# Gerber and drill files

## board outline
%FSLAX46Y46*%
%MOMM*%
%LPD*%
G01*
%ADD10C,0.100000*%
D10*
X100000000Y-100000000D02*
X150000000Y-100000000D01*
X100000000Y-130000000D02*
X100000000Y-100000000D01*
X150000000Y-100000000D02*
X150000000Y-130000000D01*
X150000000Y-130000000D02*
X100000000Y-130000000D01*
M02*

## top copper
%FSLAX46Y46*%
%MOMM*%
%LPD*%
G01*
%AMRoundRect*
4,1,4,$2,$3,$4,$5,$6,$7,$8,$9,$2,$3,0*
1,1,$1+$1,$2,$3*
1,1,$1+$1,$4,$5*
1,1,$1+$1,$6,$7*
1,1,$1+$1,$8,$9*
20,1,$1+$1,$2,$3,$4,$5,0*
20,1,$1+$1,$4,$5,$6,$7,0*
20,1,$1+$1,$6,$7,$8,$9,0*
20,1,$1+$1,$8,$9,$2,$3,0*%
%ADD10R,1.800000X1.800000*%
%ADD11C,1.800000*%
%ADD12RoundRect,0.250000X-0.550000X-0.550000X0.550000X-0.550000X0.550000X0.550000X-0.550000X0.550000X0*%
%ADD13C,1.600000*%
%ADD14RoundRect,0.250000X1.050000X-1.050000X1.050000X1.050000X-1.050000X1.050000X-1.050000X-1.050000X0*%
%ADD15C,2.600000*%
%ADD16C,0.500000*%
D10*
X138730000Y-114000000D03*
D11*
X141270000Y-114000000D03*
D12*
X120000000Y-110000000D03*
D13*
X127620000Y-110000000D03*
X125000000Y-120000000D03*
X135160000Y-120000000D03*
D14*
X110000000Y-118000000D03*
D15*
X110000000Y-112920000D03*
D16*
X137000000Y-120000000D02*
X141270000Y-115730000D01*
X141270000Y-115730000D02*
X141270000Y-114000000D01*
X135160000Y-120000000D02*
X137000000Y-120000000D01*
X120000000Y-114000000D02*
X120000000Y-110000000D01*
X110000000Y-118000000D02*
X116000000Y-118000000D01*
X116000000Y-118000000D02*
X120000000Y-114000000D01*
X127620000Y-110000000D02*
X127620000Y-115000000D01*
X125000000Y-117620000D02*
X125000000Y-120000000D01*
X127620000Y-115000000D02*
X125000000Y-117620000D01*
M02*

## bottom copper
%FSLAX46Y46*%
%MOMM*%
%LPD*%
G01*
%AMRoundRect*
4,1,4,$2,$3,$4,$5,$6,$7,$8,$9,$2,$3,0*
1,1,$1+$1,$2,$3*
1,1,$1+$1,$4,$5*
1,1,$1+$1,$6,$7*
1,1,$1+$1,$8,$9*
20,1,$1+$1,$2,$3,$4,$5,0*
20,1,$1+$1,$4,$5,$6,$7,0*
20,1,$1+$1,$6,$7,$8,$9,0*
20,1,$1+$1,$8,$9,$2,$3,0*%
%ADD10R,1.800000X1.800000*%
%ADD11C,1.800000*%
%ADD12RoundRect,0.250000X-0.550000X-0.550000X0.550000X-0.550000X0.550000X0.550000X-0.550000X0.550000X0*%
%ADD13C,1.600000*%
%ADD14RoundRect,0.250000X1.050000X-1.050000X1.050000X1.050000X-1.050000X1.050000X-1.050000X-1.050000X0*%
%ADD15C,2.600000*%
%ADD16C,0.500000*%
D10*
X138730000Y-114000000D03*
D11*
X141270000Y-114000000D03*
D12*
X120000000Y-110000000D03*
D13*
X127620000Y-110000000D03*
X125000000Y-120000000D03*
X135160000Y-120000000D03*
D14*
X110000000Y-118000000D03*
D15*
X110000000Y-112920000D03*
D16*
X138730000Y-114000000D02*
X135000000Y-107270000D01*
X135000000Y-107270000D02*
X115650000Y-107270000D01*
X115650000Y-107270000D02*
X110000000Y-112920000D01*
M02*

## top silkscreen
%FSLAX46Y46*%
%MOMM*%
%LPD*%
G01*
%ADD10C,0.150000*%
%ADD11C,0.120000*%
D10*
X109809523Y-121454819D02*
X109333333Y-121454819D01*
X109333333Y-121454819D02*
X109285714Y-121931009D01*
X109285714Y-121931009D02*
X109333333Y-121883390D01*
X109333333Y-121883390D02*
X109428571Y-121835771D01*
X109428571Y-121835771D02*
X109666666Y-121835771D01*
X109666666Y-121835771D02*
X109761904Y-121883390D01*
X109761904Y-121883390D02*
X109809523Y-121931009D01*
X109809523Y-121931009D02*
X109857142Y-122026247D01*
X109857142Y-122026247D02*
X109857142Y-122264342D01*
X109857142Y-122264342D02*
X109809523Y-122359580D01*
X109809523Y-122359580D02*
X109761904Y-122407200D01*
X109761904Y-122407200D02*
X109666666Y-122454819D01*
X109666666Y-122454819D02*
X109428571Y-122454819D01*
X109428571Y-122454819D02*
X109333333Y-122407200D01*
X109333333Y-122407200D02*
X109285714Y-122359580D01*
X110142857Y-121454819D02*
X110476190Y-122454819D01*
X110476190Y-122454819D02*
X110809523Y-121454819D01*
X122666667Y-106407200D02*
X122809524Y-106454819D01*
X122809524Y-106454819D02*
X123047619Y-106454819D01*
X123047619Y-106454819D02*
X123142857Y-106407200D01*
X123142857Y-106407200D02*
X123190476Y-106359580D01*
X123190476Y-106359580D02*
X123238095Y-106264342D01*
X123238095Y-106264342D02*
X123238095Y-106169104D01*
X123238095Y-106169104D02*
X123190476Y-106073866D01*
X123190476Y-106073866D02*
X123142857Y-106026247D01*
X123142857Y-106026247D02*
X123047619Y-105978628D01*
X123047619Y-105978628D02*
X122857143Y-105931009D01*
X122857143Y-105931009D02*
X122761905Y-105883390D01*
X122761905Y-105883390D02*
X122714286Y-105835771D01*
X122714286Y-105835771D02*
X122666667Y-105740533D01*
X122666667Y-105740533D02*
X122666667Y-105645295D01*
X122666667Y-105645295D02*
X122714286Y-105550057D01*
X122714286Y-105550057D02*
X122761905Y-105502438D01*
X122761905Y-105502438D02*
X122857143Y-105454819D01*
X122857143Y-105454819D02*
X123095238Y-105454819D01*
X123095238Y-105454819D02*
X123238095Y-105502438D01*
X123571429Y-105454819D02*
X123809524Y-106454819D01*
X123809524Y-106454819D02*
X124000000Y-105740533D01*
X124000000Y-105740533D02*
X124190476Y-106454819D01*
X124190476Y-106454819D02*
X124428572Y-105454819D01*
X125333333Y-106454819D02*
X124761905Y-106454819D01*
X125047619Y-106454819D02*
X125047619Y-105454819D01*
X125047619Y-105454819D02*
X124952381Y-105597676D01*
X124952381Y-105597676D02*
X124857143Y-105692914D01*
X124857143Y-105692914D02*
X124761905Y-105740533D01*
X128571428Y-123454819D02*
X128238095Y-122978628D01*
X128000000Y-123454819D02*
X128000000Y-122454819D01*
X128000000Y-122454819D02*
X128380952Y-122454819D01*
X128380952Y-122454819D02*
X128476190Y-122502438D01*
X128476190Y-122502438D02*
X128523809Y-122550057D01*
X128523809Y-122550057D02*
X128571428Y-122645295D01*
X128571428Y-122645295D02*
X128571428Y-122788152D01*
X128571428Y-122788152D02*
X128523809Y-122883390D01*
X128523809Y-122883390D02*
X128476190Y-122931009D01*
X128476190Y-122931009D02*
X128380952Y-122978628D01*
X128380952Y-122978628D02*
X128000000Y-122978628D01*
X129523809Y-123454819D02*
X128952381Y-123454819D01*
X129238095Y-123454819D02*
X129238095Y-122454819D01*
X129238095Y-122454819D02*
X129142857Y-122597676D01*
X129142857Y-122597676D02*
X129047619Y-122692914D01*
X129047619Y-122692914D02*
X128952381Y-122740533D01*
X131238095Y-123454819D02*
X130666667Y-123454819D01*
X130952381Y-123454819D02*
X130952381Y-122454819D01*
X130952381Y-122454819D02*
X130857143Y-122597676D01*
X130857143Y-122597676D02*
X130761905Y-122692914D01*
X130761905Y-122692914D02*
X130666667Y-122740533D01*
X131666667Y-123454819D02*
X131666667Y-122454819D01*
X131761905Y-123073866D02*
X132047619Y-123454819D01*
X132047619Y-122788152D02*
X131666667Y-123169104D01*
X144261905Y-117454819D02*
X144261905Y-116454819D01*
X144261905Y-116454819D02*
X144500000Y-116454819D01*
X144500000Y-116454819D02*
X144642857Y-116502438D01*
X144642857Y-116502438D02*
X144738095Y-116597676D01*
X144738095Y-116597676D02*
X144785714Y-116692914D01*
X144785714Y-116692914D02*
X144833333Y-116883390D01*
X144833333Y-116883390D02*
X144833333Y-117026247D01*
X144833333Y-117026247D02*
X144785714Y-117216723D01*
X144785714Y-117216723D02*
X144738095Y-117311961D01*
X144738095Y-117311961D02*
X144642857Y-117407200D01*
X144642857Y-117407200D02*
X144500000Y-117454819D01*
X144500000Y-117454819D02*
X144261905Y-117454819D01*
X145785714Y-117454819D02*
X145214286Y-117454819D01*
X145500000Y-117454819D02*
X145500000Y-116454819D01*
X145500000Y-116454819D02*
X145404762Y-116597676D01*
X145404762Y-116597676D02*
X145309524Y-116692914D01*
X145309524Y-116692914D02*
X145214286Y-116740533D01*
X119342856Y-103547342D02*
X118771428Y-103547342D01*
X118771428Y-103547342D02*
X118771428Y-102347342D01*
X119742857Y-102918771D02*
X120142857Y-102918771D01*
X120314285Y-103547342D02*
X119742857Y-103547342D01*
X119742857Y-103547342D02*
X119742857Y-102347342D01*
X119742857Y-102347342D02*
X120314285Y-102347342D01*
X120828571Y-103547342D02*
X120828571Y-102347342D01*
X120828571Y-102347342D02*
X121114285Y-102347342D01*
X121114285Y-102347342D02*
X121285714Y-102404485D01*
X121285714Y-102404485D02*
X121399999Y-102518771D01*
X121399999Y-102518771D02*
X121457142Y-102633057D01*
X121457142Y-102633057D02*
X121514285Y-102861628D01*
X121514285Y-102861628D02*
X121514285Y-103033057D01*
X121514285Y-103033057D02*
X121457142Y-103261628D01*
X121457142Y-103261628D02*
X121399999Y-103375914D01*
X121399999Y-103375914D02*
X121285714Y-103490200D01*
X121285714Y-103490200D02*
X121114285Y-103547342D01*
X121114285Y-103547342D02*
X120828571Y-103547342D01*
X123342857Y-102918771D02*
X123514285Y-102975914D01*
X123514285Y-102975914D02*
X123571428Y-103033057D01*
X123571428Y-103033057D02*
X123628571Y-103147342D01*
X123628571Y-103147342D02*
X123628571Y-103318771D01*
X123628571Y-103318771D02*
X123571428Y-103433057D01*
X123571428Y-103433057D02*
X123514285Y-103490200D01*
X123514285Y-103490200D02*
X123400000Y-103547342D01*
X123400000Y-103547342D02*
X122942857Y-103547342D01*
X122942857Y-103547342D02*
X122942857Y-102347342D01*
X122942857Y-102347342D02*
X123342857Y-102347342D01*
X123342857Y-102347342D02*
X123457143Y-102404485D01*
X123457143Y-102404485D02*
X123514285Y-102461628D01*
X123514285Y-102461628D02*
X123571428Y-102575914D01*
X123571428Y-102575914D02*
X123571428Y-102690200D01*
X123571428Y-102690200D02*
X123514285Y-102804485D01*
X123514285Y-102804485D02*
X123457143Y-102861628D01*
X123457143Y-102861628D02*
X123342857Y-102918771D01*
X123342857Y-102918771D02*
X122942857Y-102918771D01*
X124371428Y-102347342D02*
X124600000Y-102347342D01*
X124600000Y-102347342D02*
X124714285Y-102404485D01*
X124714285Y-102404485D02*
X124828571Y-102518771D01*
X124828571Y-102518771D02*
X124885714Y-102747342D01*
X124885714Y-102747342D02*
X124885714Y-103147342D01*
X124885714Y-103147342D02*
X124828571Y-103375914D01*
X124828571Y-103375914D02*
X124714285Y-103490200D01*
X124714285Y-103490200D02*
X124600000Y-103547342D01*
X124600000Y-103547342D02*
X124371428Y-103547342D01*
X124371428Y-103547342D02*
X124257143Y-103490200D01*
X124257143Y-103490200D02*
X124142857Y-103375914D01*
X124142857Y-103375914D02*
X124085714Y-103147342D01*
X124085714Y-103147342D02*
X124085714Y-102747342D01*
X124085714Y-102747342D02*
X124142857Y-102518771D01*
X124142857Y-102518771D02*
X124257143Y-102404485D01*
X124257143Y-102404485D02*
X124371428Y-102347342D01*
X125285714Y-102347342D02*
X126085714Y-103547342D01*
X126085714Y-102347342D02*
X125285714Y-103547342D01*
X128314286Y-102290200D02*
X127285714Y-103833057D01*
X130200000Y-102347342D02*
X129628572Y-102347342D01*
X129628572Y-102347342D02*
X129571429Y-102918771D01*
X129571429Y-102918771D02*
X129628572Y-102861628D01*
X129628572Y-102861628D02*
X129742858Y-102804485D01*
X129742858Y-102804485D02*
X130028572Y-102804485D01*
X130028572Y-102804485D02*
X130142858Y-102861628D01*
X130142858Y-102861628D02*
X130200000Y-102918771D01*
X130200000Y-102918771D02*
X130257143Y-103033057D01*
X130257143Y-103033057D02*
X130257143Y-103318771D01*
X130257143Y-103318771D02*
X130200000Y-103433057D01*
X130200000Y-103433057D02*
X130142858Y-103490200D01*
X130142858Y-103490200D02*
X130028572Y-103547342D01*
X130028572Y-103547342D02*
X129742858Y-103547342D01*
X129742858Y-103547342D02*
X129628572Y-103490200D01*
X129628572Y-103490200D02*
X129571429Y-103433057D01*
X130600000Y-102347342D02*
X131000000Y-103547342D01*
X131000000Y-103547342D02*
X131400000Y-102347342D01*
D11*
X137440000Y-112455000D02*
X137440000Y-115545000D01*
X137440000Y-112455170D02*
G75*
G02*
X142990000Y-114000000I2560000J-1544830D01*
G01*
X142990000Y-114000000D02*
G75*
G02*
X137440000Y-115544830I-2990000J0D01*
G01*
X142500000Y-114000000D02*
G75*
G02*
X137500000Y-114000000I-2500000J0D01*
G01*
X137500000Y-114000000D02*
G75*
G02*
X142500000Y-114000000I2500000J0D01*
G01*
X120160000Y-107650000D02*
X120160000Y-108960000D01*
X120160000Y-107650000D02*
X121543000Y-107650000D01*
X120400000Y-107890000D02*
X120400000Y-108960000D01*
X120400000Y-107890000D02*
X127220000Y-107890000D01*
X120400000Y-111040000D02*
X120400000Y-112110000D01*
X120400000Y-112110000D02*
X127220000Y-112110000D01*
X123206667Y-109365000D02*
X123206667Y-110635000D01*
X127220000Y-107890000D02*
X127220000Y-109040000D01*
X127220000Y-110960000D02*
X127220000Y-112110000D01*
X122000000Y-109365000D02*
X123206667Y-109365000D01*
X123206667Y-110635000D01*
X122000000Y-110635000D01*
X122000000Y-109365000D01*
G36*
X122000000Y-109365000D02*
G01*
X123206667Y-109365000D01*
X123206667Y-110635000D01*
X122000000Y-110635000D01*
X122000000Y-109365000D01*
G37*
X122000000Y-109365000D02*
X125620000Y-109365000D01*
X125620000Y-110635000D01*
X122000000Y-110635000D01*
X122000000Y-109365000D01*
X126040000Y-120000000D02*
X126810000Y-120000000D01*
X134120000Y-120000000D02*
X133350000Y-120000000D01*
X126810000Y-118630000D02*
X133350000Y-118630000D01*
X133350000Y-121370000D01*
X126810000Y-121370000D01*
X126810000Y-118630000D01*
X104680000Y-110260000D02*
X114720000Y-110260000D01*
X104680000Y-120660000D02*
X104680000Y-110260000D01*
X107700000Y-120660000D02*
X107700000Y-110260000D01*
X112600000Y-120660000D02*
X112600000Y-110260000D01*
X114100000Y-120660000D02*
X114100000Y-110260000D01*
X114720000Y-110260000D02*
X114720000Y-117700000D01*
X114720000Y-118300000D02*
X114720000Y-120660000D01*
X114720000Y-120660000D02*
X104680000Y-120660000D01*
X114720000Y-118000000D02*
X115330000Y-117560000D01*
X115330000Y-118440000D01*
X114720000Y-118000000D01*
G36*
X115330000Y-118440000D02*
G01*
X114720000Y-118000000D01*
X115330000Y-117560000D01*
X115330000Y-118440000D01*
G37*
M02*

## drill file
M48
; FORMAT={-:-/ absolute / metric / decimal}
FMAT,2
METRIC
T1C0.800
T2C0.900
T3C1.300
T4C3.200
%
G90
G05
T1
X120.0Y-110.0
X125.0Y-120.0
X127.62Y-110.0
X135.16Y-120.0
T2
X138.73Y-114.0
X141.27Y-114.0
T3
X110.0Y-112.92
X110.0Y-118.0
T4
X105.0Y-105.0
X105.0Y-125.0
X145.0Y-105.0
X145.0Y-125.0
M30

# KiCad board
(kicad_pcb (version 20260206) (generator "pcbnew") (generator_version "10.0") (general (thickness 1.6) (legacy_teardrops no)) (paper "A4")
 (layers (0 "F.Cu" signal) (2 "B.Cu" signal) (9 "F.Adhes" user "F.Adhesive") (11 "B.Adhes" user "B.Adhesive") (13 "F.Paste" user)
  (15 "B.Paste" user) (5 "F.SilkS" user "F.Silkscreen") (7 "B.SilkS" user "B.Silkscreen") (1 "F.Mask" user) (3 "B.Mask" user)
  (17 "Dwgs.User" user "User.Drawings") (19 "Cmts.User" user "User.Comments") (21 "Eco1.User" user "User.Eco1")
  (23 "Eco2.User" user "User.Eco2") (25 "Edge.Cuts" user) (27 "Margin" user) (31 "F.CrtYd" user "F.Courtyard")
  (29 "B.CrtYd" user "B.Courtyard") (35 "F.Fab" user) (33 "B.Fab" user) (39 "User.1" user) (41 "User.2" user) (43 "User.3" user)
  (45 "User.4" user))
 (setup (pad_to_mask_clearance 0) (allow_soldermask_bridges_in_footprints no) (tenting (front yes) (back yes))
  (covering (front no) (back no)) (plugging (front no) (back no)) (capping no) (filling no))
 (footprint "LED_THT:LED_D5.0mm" (layer "F.Cu") (at 138.73 114)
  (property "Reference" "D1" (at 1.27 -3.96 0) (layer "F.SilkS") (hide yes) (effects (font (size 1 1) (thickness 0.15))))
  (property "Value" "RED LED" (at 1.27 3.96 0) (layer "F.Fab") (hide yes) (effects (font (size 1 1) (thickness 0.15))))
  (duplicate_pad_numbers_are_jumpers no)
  (fp_line (start -1.29 -1.545) (end -1.29 1.545) (stroke (width 0.12) (type solid)) (layer "F.SilkS"))
  (fp_arc (start -1.29 -1.54483) (mid 2.071779 -2.880495) (end 4.26 0) (stroke (width 0.12) (type solid)) (layer "F.SilkS"))
  (fp_arc (start 4.26 0) (mid 2.071779 2.880495) (end -1.29 1.54483) (stroke (width 0.12) (type solid)) (layer "F.SilkS"))
  (fp_circle (center 1.27 0) (end 3.77 0) (stroke (width 0.12) (type solid)) (fill no) (layer "F.SilkS"))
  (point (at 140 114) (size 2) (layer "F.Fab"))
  (pad "1" thru_hole rect (at 0 0) (size 1.8 1.8) (drill 0.9) (layers "*.Cu" "*.Mask") (remove_unused_layers no) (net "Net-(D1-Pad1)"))
  (pad "2" thru_hole circle (at 2.54 0) (size 1.8 1.8) (drill 0.9) (layers "*.Cu" "*.Mask") (remove_unused_layers no) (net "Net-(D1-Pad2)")))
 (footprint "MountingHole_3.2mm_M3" (layer "F.Cu") (at 145 105)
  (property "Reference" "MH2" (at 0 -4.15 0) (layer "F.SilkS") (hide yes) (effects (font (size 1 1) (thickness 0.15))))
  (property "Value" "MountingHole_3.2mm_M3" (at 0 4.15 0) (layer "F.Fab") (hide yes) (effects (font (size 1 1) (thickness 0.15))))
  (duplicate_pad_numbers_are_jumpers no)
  (pad "" np_thru_hole circle (at 0 0) (size 3.2 3.2) (drill 3.2) (layers "*.Cu" "*.Mask")))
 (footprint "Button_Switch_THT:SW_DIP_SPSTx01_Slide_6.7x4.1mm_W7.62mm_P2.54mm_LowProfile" (layer "F.Cu") (at 120 110)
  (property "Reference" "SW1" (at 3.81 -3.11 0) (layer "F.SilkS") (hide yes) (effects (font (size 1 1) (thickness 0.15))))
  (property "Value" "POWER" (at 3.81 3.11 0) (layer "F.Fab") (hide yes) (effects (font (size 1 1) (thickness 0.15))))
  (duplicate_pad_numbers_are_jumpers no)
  (fp_line (start 0.16 -2.35) (end 0.16 -1.04) (stroke (width 0.12) (type solid)) (layer "F.SilkS"))
  (fp_line (start 0.16 -2.35) (end 1.543 -2.35) (stroke (width 0.12) (type solid)) (layer "F.SilkS"))
  (fp_line (start 0.4 -2.11) (end 0.4 -1.04) (stroke (width 0.12) (type solid)) (layer "F.SilkS"))
  (fp_line (start 0.4 -2.11) (end 7.22 -2.11) (stroke (width 0.12) (type solid)) (layer "F.SilkS"))
  (fp_line (start 0.4 1.04) (end 0.4 2.11) (stroke (width 0.12) (type solid)) (layer "F.SilkS"))
  (fp_line (start 0.4 2.11) (end 7.22 2.11) (stroke (width 0.12) (type solid)) (layer "F.SilkS"))
  (fp_line (start 3.206667 -0.635) (end 3.206667 0.635) (stroke (width 0.12) (type solid)) (layer "F.SilkS"))
  (fp_line (start 7.22 -2.11) (end 7.22 -0.96) (stroke (width 0.12) (type solid)) (layer "F.SilkS"))
  (fp_line (start 7.22 0.96) (end 7.22 2.11) (stroke (width 0.12) (type solid)) (layer "F.SilkS"))
  (fp_rect (start 2 -0.635) (end 3.206667 0.635) (stroke (width 0.12) (type solid)) (fill yes) (layer "F.SilkS"))
  (fp_rect (start 2 -0.635) (end 5.62 0.635) (stroke (width 0.12) (type solid)) (fill no) (layer "F.SilkS"))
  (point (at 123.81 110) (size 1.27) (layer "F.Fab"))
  (pad "1" thru_hole roundrect (at 0 0) (size 1.6 1.6) (drill 0.8) (layers "*.Cu" "*.Mask") (remove_unused_layers no)
   (roundrect_rratio 0.15625) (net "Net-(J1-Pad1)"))
  (pad "2" thru_hole circle (at 7.62 0) (size 1.6 1.6) (drill 0.8) (layers "*.Cu" "*.Mask") (remove_unused_layers no) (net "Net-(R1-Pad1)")))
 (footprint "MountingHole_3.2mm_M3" (layer "F.Cu") (at 145 125)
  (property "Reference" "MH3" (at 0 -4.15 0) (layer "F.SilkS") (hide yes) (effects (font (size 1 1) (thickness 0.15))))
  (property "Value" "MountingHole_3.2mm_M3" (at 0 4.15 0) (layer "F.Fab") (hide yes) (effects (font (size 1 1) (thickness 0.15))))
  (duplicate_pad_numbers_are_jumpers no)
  (pad "" np_thru_hole circle (at 0 0) (size 3.2 3.2) (drill 3.2) (layers "*.Cu" "*.Mask")))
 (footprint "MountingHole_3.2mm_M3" (layer "F.Cu") (at 105 125)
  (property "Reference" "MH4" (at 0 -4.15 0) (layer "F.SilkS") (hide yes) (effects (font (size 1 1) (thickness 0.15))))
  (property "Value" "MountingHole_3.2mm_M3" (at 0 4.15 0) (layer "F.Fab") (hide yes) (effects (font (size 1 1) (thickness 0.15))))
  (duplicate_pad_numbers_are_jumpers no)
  (pad "" np_thru_hole circle (at 0 0) (size 3.2 3.2) (drill 3.2) (layers "*.Cu" "*.Mask")))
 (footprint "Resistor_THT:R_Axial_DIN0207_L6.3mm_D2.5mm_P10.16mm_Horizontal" (layer "F.Cu") (at 125 120)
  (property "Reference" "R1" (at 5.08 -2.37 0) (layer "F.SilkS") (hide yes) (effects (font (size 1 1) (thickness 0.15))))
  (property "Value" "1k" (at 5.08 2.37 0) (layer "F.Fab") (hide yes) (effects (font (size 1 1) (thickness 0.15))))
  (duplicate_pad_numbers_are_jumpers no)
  (fp_line (start 1.04 0) (end 1.81 0) (stroke (width 0.12) (type solid)) (layer "F.SilkS"))
  (fp_line (start 9.12 0) (end 8.35 0) (stroke (width 0.12) (type solid)) (layer "F.SilkS"))
  (fp_rect (start 1.81 -1.37) (end 8.35 1.37) (stroke (width 0.12) (type solid)) (fill no) (layer "F.SilkS"))
  (pad "1" thru_hole circle (at 0 0) (size 1.6 1.6) (drill 0.8) (layers "*.Cu" "*.Mask") (remove_unused_layers no) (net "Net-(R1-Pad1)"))
  (pad "2" thru_hole circle (at 10.16 0) (size 1.6 1.6) (drill 0.8) (layers "*.Cu" "*.Mask") (remove_unused_layers no) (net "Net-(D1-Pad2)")))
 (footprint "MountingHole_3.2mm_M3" (layer "F.Cu") (at 105 105)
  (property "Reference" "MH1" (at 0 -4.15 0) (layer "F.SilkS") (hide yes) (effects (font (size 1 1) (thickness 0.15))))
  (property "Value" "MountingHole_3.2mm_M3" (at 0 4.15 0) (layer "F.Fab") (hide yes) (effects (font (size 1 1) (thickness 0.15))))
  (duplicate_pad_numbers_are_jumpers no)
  (pad "" np_thru_hole circle (at 0 0) (size 3.2 3.2) (drill 3.2) (layers "*.Cu" "*.Mask")))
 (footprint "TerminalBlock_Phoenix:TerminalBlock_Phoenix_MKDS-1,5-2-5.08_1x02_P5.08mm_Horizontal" (layer "F.Cu") (at 110 118 90)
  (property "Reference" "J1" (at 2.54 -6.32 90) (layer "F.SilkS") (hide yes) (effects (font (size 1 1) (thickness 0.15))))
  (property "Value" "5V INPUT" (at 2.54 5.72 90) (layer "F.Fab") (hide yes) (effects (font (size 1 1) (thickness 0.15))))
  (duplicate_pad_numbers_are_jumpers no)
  (fp_line (start 7.74 -5.32) (end 7.74 4.72) (stroke (width 0.12) (type solid)) (layer "F.SilkS"))
  (fp_line (start -2.66 -5.32) (end 7.74 -5.32) (stroke (width 0.12) (type solid)) (layer "F.SilkS"))
  (fp_line (start -2.66 -2.3) (end 7.74 -2.3) (stroke (width 0.12) (type solid)) (layer "F.SilkS"))
  (fp_line (start -2.66 2.6) (end 7.74 2.6) (stroke (width 0.12) (type solid)) (layer "F.SilkS"))
  (fp_line (start -2.66 4.1) (end 7.74 4.1) (stroke (width 0.12) (type solid)) (layer "F.SilkS"))
  (fp_line (start 7.74 4.72) (end 0.3 4.72) (stroke (width 0.12) (type solid)) (layer "F.SilkS"))
  (fp_line (start -0.3 4.72) (end -2.66 4.72) (stroke (width 0.12) (type solid)) (layer "F.SilkS"))
  (fp_line (start -2.66 4.72) (end -2.66 -5.32) (stroke (width 0.12) (type solid)) (layer "F.SilkS"))
  (fp_poly (pts (xy 0 4.72) (xy 0.44 5.33) (xy -0.44 5.33)) (stroke (width 0.12) (type solid)) (fill yes) (layer "F.SilkS"))
  (pad "1" thru_hole roundrect (at 0 0 90) (size 2.6 2.6) (drill 1.3) (layers "*.Cu" "*.Mask") (remove_unused_layers no)
   (roundrect_rratio 0.096154) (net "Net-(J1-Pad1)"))
  (pad "2" thru_hole circle (at 5.08 0 90) (size 2.6 2.6) (drill 1.3) (layers "*.Cu" "*.Mask") (remove_unused_layers no)
   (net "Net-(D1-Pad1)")))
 (gr_line (start 100 100) (end 150 100) (stroke (width 0.1) (type default)) (layer "Edge.Cuts"))
 (gr_line (start 100 130) (end 100 100) (stroke (width 0.1) (type default)) (layer "Edge.Cuts"))
 (gr_line (start 150 100) (end 150 130) (stroke (width 0.1) (type default)) (layer "Edge.Cuts"))
 (gr_line (start 150 130) (end 100 130) (stroke (width 0.1) (type default)) (layer "Edge.Cuts"))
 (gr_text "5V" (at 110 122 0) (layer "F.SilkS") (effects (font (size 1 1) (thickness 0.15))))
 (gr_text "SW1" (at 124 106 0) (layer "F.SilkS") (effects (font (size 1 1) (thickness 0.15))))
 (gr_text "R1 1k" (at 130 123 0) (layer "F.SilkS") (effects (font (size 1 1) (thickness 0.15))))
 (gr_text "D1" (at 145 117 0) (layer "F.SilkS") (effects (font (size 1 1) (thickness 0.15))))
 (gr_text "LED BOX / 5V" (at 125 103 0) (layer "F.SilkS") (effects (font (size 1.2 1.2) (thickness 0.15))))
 (segment (start 138.73 114) (end 135 107.27) (width 0.5) (layer "B.Cu") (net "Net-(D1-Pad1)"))
 (segment (start 135 107.27) (end 115.65 107.27) (width 0.5) (layer "B.Cu") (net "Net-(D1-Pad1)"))
 (segment (start 115.65 107.27) (end 110 112.92) (width 0.5) (layer "B.Cu") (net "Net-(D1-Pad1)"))
 (segment (start 137 120) (end 141.27 115.73) (width 0.5) (layer "F.Cu") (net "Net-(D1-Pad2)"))
 (segment (start 141.27 115.73) (end 141.27 114) (width 0.5) (layer "F.Cu") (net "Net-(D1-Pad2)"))
 (segment (start 135.16 120) (end 137 120) (width 0.5) (layer "F.Cu") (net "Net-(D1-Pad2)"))
 (segment (start 120 114) (end 120 110) (width 0.5) (layer "F.Cu") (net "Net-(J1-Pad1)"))
 (segment (start 110 118) (end 116 118) (width 0.5) (layer "F.Cu") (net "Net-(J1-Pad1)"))
 (segment (start 116 118) (end 120 114) (width 0.5) (layer "F.Cu") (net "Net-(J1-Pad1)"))
 (segment (start 127.62 110) (end 127.62 115) (width 0.5) (layer "F.Cu") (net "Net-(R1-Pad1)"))
 (segment (start 125 117.62) (end 125 120) (width 0.5) (layer "F.Cu") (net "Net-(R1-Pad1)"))
 (segment (start 127.62 115) (end 125 117.62) (width 0.5) (layer "F.Cu") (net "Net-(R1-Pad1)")))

